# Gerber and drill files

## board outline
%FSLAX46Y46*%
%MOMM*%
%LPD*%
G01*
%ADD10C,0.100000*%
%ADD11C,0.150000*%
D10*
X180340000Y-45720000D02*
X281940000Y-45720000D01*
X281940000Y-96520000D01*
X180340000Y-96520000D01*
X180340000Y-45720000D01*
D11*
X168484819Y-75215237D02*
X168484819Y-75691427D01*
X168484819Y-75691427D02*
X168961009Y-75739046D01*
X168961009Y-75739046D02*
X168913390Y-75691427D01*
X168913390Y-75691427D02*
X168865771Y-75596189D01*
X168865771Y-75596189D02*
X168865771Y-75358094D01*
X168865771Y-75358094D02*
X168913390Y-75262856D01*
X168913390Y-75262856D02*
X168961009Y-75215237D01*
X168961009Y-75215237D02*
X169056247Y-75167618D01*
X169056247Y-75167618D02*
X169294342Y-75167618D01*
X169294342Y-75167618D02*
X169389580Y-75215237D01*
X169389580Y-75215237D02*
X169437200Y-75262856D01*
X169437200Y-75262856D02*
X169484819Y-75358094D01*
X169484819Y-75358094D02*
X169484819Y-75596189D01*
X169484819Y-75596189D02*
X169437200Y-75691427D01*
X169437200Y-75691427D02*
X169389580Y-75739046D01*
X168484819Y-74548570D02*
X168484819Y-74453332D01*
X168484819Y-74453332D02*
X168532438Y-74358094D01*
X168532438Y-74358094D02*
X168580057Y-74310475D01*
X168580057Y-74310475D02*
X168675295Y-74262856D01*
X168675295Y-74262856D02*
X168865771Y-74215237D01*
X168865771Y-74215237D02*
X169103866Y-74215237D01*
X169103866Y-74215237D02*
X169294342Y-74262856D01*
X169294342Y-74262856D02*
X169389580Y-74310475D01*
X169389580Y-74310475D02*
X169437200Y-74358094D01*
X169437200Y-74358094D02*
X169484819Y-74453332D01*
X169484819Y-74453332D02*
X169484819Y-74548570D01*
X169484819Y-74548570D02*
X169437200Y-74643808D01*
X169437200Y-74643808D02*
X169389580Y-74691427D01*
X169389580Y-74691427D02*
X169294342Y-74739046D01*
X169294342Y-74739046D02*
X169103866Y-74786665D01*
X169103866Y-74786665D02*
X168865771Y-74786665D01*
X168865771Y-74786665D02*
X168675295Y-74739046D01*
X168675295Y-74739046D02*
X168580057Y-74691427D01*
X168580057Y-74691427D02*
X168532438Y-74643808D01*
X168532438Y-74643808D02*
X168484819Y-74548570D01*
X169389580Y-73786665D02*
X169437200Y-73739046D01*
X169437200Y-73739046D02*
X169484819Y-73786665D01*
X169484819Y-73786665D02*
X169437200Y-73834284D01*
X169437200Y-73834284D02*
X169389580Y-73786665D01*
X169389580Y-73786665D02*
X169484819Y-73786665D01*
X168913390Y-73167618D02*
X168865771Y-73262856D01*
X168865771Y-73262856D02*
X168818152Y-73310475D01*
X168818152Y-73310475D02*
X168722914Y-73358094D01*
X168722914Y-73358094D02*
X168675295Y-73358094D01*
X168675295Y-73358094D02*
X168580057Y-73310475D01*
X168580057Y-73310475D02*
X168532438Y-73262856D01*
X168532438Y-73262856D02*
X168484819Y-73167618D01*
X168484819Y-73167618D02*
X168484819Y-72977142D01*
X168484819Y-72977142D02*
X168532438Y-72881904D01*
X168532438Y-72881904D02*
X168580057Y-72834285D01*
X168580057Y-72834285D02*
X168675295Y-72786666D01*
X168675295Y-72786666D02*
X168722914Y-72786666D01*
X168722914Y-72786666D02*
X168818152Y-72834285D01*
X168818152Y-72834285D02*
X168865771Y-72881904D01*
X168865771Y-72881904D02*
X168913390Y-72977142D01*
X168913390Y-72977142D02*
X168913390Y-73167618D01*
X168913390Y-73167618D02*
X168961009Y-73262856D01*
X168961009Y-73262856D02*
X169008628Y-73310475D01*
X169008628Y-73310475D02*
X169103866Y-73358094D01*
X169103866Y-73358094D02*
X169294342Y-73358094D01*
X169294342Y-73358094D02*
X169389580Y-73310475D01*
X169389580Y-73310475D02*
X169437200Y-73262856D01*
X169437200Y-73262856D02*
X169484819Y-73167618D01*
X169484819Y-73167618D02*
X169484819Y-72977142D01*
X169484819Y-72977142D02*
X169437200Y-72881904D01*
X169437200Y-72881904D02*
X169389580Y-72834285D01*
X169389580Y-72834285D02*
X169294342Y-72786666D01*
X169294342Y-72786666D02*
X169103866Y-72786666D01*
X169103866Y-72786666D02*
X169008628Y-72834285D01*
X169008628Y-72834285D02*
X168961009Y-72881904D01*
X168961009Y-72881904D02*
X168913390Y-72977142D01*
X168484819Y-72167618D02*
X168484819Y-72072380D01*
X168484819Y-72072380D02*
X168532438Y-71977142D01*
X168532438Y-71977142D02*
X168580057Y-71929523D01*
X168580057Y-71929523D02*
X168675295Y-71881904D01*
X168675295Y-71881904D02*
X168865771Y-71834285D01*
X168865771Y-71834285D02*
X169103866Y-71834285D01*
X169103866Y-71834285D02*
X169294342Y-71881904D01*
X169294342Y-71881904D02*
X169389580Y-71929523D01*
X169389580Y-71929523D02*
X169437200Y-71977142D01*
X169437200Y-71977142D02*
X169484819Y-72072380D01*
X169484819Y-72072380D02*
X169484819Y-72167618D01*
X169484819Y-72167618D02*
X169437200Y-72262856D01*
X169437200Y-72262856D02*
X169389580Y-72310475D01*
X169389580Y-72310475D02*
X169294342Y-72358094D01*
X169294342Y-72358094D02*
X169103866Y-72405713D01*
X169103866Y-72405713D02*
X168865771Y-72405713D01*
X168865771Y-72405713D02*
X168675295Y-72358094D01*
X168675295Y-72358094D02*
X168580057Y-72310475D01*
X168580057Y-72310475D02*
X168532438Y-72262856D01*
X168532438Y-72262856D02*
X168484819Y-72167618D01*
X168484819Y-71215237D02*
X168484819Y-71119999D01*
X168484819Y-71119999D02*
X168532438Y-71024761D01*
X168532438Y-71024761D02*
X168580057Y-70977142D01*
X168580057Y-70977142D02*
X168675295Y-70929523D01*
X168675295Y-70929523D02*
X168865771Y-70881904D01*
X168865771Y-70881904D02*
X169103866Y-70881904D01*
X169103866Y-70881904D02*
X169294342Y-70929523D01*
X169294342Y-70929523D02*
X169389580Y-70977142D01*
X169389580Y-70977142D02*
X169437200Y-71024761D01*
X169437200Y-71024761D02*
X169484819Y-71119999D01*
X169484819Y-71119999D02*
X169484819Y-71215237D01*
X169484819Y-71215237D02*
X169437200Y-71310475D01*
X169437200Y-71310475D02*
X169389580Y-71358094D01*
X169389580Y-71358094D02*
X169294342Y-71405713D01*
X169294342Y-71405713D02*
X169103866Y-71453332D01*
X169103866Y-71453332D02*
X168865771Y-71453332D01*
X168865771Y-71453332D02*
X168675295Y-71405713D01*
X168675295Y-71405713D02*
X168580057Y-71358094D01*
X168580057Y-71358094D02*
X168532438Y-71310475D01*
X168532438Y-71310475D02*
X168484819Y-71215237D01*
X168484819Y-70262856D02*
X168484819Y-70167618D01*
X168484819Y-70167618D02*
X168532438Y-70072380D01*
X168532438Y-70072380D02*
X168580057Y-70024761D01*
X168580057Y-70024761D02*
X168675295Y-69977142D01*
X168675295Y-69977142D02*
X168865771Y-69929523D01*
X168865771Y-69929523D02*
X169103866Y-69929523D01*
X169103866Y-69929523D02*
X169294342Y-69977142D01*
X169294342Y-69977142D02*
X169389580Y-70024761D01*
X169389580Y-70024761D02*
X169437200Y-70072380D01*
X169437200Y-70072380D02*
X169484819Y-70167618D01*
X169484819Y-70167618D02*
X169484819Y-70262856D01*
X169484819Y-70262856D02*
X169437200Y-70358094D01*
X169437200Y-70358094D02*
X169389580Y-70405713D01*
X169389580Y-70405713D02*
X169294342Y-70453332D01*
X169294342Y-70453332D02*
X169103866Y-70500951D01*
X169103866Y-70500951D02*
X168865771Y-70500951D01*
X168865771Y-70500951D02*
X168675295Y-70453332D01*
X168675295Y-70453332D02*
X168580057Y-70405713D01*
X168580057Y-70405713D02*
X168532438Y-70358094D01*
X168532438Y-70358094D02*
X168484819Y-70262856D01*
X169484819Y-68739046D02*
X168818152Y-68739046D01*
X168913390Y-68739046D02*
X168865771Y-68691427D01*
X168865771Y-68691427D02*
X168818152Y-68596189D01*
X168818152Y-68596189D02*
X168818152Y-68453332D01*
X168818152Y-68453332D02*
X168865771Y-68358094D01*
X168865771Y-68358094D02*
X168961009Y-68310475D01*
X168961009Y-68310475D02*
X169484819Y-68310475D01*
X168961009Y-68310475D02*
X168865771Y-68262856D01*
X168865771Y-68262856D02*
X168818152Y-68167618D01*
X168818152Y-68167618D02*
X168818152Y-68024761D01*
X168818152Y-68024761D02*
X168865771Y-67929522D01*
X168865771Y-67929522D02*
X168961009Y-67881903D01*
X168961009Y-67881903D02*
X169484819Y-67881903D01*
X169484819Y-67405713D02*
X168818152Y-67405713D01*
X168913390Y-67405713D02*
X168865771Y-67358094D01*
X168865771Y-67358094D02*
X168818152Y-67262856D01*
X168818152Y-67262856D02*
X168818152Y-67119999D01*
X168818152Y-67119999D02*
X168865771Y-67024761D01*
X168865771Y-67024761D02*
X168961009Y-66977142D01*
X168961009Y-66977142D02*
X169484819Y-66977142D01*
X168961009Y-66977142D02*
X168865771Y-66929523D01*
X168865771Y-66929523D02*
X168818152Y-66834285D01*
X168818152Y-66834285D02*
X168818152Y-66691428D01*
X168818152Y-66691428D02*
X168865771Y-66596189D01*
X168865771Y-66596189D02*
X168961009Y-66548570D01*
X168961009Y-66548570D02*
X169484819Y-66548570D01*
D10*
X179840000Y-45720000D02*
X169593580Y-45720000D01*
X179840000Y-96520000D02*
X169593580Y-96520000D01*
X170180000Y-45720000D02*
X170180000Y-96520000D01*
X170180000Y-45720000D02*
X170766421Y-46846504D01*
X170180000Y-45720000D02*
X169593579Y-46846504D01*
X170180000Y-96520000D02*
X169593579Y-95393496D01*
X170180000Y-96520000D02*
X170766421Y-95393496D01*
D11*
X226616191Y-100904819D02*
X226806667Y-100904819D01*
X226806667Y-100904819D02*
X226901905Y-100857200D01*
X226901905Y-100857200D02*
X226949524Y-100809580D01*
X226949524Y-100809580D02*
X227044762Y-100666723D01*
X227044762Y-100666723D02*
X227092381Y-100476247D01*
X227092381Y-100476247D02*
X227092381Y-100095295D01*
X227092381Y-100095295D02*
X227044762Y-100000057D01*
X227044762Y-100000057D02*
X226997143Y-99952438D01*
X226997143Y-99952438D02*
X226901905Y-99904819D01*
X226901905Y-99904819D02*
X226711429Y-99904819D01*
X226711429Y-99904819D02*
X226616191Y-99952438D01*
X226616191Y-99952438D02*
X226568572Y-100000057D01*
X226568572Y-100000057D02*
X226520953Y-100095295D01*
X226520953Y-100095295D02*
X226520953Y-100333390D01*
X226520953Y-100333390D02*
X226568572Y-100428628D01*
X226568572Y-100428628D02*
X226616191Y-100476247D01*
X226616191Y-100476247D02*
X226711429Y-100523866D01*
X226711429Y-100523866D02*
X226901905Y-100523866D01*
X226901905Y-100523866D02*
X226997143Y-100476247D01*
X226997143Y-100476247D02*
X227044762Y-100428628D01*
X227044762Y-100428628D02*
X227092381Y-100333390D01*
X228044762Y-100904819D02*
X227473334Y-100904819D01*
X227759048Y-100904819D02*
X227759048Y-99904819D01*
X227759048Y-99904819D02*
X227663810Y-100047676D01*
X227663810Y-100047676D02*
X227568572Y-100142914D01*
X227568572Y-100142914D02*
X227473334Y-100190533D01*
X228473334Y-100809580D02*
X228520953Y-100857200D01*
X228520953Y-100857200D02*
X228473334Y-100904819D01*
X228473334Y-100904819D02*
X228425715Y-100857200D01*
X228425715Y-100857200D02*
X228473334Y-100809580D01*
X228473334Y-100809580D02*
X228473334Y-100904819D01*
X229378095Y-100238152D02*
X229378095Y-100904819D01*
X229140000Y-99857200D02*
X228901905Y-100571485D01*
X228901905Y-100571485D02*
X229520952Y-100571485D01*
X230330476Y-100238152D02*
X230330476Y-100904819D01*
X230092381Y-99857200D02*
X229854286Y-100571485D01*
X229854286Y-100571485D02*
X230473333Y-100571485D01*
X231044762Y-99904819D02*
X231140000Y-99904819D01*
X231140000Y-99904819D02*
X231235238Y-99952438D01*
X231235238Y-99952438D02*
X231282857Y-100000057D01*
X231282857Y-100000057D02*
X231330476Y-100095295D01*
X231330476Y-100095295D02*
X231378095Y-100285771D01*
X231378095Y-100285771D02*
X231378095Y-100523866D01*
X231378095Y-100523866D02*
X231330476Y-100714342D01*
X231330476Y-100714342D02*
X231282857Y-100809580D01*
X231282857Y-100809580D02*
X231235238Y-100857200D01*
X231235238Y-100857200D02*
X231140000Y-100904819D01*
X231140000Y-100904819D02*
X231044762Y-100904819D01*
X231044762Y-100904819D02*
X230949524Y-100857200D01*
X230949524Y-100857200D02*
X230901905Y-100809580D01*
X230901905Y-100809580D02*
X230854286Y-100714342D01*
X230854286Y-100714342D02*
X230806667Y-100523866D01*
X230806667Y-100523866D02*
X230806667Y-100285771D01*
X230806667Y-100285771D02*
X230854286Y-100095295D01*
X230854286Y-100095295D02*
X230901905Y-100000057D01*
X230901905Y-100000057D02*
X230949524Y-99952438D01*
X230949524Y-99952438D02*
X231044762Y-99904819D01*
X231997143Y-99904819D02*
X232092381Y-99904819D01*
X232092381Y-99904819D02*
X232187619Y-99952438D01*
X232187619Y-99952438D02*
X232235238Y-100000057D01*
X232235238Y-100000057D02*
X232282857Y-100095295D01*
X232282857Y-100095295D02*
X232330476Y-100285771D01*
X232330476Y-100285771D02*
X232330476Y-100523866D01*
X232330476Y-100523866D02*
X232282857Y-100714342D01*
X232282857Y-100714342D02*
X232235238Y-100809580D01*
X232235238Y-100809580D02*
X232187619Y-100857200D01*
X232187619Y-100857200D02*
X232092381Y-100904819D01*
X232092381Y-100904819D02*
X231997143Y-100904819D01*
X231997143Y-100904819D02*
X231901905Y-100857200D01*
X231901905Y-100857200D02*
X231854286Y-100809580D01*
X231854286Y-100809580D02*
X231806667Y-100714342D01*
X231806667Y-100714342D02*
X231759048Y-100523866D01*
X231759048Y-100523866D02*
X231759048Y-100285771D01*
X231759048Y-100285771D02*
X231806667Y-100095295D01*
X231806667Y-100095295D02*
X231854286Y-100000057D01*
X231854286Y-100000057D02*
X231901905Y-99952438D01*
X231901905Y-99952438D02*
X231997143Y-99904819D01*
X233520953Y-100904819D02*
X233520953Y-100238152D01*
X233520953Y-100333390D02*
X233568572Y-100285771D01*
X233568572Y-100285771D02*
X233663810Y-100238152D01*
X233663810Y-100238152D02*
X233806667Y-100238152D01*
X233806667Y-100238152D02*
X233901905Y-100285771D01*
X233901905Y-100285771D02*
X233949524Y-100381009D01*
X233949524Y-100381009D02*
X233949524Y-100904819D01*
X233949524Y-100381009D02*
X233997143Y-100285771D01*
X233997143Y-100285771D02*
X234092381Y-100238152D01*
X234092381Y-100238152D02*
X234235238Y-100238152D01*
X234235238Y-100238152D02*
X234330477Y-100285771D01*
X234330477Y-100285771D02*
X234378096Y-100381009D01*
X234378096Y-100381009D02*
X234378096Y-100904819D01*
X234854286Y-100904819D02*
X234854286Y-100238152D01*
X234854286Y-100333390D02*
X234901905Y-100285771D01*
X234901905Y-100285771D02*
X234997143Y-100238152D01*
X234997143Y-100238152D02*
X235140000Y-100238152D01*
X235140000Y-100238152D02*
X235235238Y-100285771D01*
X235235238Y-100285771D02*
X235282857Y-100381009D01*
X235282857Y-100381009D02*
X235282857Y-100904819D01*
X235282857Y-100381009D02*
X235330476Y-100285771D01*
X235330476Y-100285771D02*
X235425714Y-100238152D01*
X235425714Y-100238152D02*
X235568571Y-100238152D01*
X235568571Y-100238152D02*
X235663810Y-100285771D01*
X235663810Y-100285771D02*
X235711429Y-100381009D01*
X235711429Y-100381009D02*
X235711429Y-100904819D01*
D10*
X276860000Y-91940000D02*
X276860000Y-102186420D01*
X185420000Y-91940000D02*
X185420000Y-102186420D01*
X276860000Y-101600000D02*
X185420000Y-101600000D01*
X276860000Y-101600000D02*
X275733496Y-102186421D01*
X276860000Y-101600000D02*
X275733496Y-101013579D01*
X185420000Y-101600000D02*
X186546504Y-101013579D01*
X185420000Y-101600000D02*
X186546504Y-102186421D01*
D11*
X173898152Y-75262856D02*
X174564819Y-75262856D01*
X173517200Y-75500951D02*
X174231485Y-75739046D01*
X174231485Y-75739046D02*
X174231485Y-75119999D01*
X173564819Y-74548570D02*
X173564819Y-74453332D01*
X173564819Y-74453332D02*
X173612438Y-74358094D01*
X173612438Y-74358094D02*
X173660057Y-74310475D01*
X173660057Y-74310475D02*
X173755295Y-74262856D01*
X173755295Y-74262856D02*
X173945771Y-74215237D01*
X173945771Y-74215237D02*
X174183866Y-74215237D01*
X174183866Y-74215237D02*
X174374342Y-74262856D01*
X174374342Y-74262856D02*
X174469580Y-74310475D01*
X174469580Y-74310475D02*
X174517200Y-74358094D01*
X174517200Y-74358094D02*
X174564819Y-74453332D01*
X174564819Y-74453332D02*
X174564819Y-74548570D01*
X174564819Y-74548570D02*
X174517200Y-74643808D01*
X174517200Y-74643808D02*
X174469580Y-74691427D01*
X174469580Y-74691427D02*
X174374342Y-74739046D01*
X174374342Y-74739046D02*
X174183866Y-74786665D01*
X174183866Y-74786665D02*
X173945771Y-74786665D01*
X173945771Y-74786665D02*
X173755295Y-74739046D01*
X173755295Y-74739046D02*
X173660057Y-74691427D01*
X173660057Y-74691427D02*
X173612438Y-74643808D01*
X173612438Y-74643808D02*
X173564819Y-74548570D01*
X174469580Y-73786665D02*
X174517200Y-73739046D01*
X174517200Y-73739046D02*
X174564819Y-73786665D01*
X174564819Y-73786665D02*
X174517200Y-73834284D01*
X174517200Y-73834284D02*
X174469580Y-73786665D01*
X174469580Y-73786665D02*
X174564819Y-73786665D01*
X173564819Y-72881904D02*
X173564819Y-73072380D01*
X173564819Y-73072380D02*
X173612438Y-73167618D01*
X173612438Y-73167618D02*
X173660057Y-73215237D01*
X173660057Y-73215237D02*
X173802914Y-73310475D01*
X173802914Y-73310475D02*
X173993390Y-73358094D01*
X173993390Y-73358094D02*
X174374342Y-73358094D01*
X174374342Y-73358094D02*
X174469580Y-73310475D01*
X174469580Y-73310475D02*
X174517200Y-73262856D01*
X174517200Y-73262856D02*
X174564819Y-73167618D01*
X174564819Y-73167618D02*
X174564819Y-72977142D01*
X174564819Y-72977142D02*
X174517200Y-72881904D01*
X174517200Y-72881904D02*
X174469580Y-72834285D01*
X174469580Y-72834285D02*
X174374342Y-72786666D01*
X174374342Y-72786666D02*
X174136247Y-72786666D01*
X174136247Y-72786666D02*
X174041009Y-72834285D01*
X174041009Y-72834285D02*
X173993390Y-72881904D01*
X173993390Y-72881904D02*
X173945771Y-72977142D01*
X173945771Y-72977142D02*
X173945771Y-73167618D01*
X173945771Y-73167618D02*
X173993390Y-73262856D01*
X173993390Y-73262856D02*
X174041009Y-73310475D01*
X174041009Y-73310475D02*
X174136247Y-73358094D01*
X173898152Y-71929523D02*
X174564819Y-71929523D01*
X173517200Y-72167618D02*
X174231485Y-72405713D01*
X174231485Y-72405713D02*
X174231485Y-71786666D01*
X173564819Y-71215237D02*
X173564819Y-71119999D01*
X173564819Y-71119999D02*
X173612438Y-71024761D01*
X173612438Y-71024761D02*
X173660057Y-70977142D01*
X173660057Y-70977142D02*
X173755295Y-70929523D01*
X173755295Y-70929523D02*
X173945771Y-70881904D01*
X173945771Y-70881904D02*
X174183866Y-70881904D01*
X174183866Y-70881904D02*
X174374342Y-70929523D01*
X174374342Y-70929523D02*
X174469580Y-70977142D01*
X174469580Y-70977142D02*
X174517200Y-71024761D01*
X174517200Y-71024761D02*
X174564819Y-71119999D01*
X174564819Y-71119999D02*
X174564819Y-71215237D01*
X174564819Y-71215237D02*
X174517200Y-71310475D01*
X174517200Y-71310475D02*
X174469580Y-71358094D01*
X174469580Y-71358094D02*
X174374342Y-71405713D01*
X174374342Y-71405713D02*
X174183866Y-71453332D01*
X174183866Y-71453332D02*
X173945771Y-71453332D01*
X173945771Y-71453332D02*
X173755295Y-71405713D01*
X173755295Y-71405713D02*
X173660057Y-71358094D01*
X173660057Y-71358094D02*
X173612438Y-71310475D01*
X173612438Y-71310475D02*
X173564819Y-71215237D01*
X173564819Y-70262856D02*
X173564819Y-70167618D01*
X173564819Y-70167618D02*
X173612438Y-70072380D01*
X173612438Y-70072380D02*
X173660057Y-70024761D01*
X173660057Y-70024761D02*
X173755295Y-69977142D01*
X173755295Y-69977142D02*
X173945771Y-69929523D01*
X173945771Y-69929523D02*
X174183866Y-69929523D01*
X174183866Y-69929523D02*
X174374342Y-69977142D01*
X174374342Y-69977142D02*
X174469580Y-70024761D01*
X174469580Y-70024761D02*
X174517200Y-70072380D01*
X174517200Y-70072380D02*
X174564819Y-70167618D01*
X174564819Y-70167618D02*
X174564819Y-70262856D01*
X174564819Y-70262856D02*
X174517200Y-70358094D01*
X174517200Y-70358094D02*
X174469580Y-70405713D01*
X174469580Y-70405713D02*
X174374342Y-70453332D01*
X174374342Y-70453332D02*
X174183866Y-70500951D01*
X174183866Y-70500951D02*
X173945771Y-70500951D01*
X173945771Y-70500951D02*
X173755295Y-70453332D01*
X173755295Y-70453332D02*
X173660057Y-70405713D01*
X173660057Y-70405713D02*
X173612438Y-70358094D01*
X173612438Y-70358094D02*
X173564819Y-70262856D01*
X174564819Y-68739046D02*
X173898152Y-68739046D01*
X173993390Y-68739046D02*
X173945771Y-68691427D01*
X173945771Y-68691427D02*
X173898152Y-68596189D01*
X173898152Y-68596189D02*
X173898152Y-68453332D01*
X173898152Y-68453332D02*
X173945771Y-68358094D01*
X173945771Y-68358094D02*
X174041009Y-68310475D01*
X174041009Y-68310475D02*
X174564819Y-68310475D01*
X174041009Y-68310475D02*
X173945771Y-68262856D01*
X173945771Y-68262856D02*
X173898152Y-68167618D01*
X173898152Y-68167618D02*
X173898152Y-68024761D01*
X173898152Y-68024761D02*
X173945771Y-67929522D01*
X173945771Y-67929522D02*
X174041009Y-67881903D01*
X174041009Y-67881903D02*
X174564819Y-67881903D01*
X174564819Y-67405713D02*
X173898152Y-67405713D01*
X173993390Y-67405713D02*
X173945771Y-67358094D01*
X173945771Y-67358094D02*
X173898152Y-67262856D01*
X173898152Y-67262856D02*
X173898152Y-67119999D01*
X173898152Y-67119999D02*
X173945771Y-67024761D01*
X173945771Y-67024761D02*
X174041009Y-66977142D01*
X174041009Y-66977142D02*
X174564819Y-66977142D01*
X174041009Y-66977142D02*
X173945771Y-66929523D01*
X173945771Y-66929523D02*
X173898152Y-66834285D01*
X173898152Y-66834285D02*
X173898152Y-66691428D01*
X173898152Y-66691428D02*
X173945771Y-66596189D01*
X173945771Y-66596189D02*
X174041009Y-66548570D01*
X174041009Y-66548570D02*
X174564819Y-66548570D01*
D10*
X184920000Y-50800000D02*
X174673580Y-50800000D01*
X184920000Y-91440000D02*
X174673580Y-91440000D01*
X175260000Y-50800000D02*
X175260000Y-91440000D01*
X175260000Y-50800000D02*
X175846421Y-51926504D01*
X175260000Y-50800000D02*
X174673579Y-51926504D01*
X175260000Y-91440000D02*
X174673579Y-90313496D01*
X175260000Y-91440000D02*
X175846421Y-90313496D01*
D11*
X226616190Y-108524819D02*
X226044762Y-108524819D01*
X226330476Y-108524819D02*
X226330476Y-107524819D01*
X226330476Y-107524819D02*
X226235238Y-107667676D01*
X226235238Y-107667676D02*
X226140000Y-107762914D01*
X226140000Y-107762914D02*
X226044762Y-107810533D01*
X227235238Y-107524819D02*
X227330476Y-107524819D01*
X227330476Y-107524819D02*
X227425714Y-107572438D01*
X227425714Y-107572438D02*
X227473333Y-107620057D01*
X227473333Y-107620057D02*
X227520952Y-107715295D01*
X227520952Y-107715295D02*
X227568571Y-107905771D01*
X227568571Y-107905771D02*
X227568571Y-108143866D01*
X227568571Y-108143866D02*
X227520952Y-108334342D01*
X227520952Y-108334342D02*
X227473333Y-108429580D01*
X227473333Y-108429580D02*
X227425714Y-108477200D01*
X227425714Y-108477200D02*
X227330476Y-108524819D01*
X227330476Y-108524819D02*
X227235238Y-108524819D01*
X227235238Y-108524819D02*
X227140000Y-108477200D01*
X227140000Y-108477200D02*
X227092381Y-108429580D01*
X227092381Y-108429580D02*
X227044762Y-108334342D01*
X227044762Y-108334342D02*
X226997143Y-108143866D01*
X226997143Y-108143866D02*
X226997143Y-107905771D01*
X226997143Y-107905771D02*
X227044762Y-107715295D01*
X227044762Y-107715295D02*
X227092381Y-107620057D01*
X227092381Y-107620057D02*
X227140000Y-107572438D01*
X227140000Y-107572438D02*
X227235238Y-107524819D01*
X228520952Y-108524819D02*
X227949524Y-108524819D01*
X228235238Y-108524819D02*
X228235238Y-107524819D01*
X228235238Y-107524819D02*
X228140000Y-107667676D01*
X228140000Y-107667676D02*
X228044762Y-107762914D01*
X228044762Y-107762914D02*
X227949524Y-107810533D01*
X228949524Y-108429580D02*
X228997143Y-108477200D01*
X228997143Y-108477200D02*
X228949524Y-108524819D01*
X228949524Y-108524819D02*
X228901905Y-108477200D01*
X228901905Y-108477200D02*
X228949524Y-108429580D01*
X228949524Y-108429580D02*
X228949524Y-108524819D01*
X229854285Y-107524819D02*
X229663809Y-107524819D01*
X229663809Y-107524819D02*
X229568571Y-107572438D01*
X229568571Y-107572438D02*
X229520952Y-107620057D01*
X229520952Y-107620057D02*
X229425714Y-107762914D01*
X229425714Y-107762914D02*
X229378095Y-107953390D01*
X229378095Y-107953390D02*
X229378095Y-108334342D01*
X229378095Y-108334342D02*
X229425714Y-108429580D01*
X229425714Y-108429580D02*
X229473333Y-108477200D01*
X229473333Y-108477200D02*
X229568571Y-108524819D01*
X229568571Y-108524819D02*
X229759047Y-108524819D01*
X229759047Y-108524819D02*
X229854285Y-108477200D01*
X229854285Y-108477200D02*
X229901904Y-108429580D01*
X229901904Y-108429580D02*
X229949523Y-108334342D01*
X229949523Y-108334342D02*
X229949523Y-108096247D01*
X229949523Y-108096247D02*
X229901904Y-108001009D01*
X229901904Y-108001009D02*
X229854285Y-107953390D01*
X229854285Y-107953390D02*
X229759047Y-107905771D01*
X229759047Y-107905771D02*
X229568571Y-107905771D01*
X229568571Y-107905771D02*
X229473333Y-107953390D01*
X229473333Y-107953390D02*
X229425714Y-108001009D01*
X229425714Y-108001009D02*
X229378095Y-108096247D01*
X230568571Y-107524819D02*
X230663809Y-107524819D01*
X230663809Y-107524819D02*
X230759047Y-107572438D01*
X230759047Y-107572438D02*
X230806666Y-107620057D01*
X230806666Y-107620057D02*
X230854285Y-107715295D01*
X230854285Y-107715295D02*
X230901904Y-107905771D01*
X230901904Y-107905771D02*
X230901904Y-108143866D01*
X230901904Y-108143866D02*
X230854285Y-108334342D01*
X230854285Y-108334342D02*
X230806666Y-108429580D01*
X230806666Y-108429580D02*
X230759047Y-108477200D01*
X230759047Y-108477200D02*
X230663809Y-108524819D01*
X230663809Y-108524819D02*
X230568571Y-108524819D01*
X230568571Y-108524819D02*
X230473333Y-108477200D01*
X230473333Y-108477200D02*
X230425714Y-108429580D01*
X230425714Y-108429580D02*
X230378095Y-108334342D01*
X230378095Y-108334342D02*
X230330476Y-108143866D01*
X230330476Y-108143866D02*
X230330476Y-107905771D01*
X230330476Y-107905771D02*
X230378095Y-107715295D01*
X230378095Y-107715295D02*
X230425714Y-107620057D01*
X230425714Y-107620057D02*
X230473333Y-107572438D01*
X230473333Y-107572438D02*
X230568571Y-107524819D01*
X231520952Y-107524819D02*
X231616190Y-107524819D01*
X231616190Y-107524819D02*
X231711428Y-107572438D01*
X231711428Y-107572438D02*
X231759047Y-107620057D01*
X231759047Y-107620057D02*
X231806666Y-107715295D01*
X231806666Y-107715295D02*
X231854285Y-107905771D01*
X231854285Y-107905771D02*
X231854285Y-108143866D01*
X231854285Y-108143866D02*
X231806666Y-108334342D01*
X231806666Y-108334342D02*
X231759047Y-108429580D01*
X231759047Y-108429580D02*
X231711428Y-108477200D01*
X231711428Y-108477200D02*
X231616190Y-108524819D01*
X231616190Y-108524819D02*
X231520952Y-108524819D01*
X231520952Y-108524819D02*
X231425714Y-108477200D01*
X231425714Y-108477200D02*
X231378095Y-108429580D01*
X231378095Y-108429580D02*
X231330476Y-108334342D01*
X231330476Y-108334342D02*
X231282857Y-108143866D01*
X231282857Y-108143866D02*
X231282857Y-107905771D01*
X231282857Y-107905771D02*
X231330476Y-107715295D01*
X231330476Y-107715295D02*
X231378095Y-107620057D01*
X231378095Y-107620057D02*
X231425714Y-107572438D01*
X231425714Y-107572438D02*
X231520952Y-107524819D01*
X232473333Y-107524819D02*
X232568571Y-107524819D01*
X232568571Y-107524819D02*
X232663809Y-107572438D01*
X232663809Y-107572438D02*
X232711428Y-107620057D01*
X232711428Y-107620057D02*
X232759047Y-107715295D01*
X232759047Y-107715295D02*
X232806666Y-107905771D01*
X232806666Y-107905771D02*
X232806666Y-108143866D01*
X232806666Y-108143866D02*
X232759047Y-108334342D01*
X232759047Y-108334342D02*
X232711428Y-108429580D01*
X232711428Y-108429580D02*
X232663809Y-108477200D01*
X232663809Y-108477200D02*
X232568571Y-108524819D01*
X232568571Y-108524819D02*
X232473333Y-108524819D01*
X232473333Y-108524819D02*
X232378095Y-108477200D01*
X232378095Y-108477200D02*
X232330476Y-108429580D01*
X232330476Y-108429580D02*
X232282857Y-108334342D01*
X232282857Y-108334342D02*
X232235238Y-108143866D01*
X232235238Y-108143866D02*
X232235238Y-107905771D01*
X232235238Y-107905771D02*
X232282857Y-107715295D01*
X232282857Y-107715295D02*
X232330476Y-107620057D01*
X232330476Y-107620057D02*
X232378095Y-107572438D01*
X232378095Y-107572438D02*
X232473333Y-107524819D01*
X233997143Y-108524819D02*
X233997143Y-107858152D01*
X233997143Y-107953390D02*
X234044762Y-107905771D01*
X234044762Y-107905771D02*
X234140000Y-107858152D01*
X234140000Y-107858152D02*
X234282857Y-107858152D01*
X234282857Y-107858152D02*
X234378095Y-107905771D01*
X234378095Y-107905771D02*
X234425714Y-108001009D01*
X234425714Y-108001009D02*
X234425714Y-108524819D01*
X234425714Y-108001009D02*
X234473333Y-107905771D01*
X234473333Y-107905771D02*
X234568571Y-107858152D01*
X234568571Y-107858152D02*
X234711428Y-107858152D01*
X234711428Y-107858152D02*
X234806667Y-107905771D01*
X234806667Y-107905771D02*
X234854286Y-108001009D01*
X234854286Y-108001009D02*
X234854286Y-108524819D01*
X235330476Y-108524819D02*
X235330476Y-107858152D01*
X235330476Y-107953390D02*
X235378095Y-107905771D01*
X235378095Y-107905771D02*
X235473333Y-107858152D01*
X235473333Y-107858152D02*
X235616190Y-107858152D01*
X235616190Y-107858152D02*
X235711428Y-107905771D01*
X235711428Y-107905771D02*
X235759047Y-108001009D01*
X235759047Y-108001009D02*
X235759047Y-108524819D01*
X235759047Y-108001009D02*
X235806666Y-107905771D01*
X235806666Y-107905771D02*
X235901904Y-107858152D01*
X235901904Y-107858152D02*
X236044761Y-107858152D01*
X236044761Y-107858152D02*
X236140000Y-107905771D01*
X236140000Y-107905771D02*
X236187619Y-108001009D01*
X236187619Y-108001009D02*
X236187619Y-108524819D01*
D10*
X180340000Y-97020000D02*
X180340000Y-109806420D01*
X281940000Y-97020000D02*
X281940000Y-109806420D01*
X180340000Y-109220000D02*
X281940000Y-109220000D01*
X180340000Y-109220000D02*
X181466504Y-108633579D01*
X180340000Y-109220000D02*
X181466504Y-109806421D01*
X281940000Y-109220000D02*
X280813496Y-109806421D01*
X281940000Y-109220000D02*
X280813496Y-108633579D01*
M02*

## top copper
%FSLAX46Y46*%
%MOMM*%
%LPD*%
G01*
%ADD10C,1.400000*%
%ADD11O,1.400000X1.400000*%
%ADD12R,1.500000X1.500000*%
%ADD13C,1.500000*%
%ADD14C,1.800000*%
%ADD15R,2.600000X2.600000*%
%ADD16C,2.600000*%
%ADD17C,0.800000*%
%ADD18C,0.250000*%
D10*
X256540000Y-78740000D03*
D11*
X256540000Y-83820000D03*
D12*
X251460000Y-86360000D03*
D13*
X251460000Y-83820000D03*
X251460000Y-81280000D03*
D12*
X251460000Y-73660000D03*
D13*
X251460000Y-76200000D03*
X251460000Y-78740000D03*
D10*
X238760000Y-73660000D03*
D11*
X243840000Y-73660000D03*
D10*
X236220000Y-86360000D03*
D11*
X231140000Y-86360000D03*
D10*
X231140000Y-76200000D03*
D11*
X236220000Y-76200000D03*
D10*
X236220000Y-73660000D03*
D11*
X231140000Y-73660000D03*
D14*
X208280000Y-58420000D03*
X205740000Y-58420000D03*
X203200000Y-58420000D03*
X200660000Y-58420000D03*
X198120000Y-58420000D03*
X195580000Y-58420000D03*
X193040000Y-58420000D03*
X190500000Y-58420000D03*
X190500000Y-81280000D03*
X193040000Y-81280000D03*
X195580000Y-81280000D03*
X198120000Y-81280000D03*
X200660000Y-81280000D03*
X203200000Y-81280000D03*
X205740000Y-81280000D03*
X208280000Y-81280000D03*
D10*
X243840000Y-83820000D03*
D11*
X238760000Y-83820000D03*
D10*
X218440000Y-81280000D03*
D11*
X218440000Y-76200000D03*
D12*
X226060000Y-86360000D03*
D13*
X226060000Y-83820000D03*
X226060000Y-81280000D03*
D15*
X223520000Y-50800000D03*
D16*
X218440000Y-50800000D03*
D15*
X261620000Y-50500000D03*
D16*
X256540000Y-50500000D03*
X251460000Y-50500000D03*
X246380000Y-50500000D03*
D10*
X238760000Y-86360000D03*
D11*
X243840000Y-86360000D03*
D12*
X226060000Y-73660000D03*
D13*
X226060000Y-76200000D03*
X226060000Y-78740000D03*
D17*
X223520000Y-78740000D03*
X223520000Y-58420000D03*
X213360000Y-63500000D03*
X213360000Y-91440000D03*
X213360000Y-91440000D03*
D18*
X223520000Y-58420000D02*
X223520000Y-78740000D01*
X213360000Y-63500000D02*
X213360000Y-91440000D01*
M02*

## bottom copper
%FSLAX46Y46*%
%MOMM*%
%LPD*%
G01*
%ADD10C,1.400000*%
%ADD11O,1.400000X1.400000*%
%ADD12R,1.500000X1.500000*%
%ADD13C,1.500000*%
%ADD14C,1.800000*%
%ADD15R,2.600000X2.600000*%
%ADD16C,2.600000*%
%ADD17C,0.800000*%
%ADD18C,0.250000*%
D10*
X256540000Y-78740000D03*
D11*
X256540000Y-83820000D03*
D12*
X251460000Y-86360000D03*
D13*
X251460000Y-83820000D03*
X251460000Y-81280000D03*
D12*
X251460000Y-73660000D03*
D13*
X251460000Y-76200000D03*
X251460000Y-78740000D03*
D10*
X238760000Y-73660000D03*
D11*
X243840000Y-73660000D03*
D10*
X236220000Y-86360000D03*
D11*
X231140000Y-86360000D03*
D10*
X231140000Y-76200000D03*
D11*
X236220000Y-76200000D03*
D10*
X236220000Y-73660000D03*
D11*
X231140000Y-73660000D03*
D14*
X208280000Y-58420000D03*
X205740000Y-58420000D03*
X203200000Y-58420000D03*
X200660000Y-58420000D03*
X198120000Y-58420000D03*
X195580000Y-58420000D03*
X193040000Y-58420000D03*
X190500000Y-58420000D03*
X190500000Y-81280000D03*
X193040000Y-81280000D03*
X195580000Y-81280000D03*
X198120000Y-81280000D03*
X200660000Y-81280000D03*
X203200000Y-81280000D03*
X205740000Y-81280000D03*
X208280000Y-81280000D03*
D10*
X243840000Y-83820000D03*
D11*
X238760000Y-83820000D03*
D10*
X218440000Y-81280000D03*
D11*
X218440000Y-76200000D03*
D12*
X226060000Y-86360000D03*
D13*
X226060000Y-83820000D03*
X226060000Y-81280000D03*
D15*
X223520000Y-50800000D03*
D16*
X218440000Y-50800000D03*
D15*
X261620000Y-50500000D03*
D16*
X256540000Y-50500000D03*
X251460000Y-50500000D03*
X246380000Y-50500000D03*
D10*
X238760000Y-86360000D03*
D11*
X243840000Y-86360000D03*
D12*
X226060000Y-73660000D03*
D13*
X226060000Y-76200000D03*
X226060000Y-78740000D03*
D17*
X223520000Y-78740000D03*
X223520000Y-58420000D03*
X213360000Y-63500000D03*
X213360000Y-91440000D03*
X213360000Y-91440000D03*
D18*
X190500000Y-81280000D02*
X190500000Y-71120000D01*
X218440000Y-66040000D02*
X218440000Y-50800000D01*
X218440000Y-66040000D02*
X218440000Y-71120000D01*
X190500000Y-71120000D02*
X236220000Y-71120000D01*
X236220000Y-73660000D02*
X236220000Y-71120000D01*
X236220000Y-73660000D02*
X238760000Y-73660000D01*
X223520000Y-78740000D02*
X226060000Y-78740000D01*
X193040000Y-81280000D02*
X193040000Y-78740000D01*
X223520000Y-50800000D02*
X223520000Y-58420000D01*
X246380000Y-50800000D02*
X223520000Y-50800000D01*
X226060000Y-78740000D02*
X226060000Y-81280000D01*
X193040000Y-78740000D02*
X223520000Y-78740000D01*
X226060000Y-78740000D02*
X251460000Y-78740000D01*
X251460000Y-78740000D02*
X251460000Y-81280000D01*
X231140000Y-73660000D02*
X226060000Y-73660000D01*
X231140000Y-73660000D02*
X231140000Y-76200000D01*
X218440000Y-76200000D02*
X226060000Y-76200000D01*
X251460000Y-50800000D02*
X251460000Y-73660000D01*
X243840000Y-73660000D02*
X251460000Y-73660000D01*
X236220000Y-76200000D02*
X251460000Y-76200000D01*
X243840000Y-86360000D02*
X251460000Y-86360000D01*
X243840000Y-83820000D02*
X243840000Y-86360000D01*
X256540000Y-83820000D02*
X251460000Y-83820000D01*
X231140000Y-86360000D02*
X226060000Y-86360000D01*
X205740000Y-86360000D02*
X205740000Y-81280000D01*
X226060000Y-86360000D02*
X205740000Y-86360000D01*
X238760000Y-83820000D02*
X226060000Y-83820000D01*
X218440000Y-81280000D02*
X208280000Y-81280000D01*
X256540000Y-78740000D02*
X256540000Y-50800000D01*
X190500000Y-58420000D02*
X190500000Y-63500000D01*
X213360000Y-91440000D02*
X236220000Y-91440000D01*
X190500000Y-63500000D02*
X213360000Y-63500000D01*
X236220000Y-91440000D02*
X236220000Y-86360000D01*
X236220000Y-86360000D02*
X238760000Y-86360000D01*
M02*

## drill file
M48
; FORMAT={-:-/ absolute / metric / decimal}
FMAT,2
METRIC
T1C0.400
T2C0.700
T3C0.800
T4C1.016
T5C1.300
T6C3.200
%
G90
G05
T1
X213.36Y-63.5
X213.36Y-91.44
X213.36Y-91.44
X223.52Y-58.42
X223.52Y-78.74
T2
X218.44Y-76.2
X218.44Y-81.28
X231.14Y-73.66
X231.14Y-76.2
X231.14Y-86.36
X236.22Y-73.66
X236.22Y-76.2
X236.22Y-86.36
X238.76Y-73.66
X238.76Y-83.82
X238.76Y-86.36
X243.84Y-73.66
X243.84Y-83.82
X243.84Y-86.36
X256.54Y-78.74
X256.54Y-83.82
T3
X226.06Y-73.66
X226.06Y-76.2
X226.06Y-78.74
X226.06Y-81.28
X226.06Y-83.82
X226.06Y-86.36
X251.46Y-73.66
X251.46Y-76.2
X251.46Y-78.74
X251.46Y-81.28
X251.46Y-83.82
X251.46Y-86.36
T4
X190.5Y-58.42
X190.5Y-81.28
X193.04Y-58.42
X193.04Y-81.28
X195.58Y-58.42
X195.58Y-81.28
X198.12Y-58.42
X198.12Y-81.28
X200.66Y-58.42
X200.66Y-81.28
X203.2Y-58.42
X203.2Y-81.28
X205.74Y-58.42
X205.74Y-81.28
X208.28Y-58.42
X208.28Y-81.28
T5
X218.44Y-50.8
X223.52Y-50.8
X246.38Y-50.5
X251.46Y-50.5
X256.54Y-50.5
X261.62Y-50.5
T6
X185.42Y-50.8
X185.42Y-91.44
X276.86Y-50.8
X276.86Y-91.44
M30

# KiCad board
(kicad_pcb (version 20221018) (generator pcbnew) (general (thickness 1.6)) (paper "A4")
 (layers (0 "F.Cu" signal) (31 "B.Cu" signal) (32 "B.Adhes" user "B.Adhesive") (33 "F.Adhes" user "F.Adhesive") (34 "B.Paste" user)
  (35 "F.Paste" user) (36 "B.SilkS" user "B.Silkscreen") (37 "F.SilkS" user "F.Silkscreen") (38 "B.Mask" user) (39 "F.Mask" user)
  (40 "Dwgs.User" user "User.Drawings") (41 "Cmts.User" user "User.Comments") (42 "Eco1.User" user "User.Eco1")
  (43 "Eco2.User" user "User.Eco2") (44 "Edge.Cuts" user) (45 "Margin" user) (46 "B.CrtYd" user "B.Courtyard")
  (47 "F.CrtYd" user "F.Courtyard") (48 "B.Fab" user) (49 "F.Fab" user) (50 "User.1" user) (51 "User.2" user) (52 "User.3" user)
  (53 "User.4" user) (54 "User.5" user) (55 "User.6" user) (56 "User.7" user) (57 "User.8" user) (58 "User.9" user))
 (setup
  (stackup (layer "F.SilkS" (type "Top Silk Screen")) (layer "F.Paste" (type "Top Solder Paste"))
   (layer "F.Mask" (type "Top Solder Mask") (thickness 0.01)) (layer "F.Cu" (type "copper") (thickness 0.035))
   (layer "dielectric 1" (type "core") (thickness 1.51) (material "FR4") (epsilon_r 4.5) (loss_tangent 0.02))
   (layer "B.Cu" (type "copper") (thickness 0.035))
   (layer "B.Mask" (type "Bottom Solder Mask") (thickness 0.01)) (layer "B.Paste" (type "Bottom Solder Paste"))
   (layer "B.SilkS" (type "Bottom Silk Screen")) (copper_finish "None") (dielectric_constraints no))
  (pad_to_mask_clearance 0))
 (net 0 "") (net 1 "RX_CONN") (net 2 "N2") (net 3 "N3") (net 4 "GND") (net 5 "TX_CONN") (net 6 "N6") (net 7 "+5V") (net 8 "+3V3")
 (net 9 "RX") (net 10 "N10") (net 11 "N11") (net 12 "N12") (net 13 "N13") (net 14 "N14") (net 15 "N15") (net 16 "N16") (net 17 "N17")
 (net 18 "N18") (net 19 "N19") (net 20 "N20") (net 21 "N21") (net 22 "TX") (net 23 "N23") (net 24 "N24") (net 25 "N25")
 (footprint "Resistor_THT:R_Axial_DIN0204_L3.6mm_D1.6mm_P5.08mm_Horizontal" (layer "F.Cu") (at 256.54 78.74 -90)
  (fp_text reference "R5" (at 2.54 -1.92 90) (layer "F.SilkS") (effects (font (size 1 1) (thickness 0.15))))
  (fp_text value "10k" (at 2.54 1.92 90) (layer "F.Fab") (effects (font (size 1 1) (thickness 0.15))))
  (pad "1" thru_hole circle (at 0 0 270) (size 1.4 1.4) (drill 0.7) (layers "*.Cu" "*.Mask") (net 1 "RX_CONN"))
  (pad "2" thru_hole oval (at 5.08 0 270) (size 1.4 1.4) (drill 0.7) (layers "*.Cu" "*.Mask") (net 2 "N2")))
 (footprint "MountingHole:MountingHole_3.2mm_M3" (layer "F.Cu") (at 185.42 91.44)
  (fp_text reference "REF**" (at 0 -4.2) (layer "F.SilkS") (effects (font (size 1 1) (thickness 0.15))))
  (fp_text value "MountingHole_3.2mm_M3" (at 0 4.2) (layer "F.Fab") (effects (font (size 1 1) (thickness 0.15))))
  (pad "" np_thru_hole circle (at 0 0) (size 3.2 3.2) (drill 3.2) (layers "*.Cu" "*.Mask")))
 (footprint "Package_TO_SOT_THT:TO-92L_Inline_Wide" (layer "F.Cu") (at 251.46 86.36 90)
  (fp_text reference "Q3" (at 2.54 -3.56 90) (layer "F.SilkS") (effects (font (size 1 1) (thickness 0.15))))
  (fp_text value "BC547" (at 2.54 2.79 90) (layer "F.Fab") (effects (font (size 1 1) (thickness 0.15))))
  (pad "1" thru_hole rect (at 0 0 90) (size 1.5 1.5) (drill 0.8) (layers "*.Cu" "*.Mask") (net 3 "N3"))
  (pad "2" thru_hole circle (at 2.54 0 90) (size 1.5 1.5) (drill 0.8) (layers "*.Cu" "*.Mask") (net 2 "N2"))
  (pad "3" thru_hole circle (at 5.08 0 90) (size 1.5 1.5) (drill 0.8) (layers "*.Cu" "*.Mask") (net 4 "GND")))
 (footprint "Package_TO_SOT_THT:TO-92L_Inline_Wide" (layer "F.Cu") (at 251.46 73.66 -90)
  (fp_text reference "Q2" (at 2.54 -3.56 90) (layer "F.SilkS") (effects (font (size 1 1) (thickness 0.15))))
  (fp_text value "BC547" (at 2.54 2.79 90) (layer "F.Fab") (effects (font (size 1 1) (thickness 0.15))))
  (pad "1" thru_hole rect (at 0 0 270) (size 1.5 1.5) (drill 0.8) (layers "*.Cu" "*.Mask") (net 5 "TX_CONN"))
  (pad "2" thru_hole circle (at 2.54 0 270) (size 1.5 1.5) (drill 0.8) (layers "*.Cu" "*.Mask") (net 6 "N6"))
  (pad "3" thru_hole circle (at 5.08 0 270) (size 1.5 1.5) (drill 0.8) (layers "*.Cu" "*.Mask") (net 4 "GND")))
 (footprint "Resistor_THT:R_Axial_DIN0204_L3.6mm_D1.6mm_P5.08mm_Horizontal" (layer "F.Cu") (at 238.76 73.66)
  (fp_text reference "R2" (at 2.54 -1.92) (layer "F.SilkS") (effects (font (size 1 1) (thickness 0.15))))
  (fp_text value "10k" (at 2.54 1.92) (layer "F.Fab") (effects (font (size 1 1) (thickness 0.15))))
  (pad "1" thru_hole circle (at 0 0) (size 1.4 1.4) (drill 0.7) (layers "*.Cu" "*.Mask") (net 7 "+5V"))
  (pad "2" thru_hole oval (at 5.08 0) (size 1.4 1.4) (drill 0.7) (layers "*.Cu" "*.Mask") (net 5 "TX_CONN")))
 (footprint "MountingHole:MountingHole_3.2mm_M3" (layer "F.Cu") (at 276.86 91.44)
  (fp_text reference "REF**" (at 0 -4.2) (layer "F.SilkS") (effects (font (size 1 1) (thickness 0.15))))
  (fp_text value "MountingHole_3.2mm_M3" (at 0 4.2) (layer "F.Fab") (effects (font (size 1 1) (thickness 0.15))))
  (pad "" np_thru_hole circle (at 0 0) (size 3.2 3.2) (drill 3.2) (layers "F&B.Cu" "*.Mask")))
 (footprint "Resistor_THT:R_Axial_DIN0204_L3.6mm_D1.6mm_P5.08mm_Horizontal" (layer "F.Cu") (at 236.22 86.36 180)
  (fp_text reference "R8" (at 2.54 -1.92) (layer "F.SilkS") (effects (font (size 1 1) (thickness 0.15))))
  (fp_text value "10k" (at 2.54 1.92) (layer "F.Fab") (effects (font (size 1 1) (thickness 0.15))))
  (pad "1" thru_hole circle (at 0 0 180) (size 1.4 1.4) (drill 0.7) (layers "*.Cu" "*.Mask") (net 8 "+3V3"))
  (pad "2" thru_hole oval (at 5.08 0 180) (size 1.4 1.4) (drill 0.7) (layers "*.Cu" "*.Mask") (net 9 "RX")))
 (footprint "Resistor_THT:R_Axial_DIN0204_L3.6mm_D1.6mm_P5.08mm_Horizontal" (layer "F.Cu") (at 231.14 76.2)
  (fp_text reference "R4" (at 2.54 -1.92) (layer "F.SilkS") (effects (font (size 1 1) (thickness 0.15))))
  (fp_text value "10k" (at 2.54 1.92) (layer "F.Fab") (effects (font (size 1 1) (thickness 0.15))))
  (pad "1" thru_hole circle (at 0 0) (size 1.4 1.4) (drill 0.7) (layers "*.Cu" "*.Mask") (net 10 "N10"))
  (pad "2" thru_hole oval (at 5.08 0) (size 1.4 1.4) (drill 0.7) (layers "*.Cu" "*.Mask") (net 6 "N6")))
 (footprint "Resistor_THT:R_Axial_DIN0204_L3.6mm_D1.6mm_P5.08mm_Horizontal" (layer "F.Cu") (at 236.22 73.66 180)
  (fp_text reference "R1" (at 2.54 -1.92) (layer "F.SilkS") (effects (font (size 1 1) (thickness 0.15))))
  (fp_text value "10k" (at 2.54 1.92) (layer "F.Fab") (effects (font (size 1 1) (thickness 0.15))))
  (pad "1" thru_hole circle (at 0 0 180) (size 1.4 1.4) (drill 0.7) (layers "*.Cu" "*.Mask") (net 7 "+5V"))
  (pad "2" thru_hole oval (at 5.08 0 180) (size 1.4 1.4) (drill 0.7) (layers "*.Cu" "*.Mask") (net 10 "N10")))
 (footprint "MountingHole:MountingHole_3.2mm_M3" (layer "F.Cu") (at 185.42 50.8)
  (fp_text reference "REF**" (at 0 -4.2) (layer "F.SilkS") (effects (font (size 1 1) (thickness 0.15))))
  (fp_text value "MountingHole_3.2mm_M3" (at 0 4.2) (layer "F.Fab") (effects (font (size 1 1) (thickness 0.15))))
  (pad "" np_thru_hole circle (at 0 0) (size 3.2 3.2) (drill 3.2) (layers "F&B.Cu" "*.Mask")))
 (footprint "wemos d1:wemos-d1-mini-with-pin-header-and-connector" (layer "F.Cu") (at 199.39 69.85)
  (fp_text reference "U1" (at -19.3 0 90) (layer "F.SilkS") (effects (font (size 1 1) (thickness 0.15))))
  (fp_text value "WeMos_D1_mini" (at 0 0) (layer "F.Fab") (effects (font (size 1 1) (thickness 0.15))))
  (pad "1" thru_hole circle (at 8.89 -11.43) (size 1.8 1.8) (drill 1.016) (layers "*.Cu" "*.Mask") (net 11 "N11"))
  (pad "2" thru_hole circle (at 6.35 -11.43) (size 1.8 1.8) (drill 1.016) (layers "*.Cu" "*.Mask") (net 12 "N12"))
  (pad "3" thru_hole circle (at 3.81 -11.43) (size 1.8 1.8) (drill 1.016) (layers "*.Cu" "*.Mask") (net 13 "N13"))
  (pad "4" thru_hole circle (at 1.27 -11.43) (size 1.8 1.8) (drill 1.016) (layers "*.Cu" "*.Mask") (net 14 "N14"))
  (pad "5" thru_hole circle (at -1.27 -11.43) (size 1.8 1.8) (drill 1.016) (layers "*.Cu" "*.Mask") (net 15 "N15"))
  (pad "6" thru_hole circle (at -3.81 -11.43 90) (size 1.8 1.8) (drill 1.016) (layers "*.Cu" "*.Mask") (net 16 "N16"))
  (pad "7" thru_hole circle (at -6.35 -11.43) (size 1.8 1.8) (drill 1.016) (layers "*.Cu" "*.Mask") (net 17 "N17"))
  (pad "8" thru_hole circle (at -8.89 -11.43) (size 1.8 1.8) (drill 1.016) (layers "*.Cu" "*.Mask") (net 8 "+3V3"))
  (pad "9" thru_hole circle (at -8.89 11.43) (size 1.8 1.8) (drill 1.016) (layers "*.Cu" "*.Mask") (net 7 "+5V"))
  (pad "10" thru_hole circle (at -6.35 11.43) (size 1.8 1.8) (drill 1.016) (layers "*.Cu" "*.Mask") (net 4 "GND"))
  (pad "11" thru_hole circle (at -3.81 11.43) (size 1.8 1.8) (drill 1.016) (layers "*.Cu" "*.Mask") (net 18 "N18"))
  (pad "12" thru_hole circle (at -1.27 11.43) (size 1.8 1.8) (drill 1.016) (layers "*.Cu" "*.Mask") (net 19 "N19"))
  (pad "13" thru_hole circle (at 1.27 11.43) (size 1.8 1.8) (drill 1.016) (layers "*.Cu" "*.Mask") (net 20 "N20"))
  (pad "14" thru_hole circle (at 3.81 11.43) (size 1.8 1.8) (drill 1.016) (layers "*.Cu" "*.Mask") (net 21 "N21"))
  (pad "15" thru_hole circle (at 6.35 11.43) (size 1.8 1.8) (drill 1.016) (layers "*.Cu" "*.Mask") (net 9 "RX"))
  (pad "16" thru_hole circle (at 8.89 11.43) (size 1.8 1.8) (drill 1.016) (layers "*.Cu" "*.Mask") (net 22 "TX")))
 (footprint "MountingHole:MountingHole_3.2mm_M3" (layer "F.Cu") (at 276.86 50.8)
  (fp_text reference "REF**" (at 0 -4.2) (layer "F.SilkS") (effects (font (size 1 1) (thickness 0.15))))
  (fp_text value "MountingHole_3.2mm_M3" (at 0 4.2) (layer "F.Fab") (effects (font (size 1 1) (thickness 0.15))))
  (pad "" np_thru_hole circle (at 0 0) (size 3.2 3.2) (drill 3.2) (layers "F&B.Cu" "*.Mask")))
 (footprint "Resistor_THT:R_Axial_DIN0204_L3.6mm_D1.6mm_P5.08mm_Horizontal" (layer "F.Cu") (at 243.84 83.82 180)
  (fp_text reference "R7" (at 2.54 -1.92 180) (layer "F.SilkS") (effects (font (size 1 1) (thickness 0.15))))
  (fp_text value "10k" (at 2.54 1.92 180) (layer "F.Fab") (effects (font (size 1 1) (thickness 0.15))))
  (pad "1" thru_hole circle (at 0 0 180) (size 1.4 1.4) (drill 0.7) (layers "*.Cu" "*.Mask") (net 3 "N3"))
  (pad "2" thru_hole oval (at 5.08 0 180) (size 1.4 1.4) (drill 0.7) (layers "*.Cu" "*.Mask") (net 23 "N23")))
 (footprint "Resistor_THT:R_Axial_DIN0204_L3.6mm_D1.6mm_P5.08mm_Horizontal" (layer "F.Cu") (at 218.44 81.28 90)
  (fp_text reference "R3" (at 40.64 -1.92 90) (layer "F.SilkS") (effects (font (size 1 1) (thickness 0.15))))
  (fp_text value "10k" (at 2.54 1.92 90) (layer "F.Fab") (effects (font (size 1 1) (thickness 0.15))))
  (pad "1" thru_hole circle (at 0 0 90) (size 1.4 1.4) (drill 0.7) (layers "*.Cu" "*.Mask") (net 22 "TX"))
  (pad "2" thru_hole oval (at 5.08 0 90) (size 1.4 1.4) (drill 0.7) (layers "*.Cu" "*.Mask") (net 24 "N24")))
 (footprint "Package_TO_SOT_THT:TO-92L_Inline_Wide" (layer "F.Cu") (at 226.06 86.36 90)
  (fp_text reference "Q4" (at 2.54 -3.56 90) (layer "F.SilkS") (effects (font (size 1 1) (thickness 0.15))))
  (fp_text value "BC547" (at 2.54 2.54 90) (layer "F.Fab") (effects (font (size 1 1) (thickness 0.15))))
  (pad "1" thru_hole rect (at 0 0 90) (size 1.5 1.5) (drill 0.8) (layers "*.Cu" "*.Mask") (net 9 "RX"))
  (pad "2" thru_hole circle (at 2.54 0 90) (size 1.5 1.5) (drill 0.8) (layers "*.Cu" "*.Mask") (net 23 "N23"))
  (pad "3" thru_hole circle (at 5.08 0 90) (size 1.5 1.5) (drill 0.8) (layers "*.Cu" "*.Mask") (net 4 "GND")))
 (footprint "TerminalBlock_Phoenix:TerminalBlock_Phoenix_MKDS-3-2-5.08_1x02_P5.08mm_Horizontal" (layer "F.Cu") (at 223.52 50.8 180)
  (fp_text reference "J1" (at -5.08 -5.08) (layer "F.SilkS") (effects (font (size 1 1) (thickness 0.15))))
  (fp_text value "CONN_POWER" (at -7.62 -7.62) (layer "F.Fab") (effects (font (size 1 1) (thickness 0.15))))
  (pad "1" thru_hole rect (at 0 0 180) (size 2.6 2.6) (drill 1.3) (layers "*.Cu" "*.Mask") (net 4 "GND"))
  (pad "2" thru_hole circle (at 5.08 0 180) (size 2.6 2.6) (drill 1.3) (layers "*.Cu" "*.Mask") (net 7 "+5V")))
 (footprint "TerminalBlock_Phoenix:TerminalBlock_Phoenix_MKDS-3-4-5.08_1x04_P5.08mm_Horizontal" (layer "F.Cu") (at 261.62 50.5 180)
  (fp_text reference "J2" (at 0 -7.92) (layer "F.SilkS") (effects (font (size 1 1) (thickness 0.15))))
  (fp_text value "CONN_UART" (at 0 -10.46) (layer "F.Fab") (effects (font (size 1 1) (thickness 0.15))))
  (pad "1" thru_hole rect (at 0 0 180) (size 2.6 2.6) (drill 1.3) (layers "*.Cu" "*.Mask") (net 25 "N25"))
  (pad "2" thru_hole circle (at 5.08 0 180) (size 2.6 2.6) (drill 1.3) (layers "*.Cu" "*.Mask") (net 1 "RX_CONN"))
  (pad "3" thru_hole circle (at 10.16 0 180) (size 2.6 2.6) (drill 1.3) (layers "*.Cu" "*.Mask") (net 5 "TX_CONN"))
  (pad "4" thru_hole circle (at 15.24 0 180) (size 2.6 2.6) (drill 1.3) (layers "*.Cu" "*.Mask") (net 4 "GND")))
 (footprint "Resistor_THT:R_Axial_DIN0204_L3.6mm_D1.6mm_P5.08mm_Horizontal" (layer "F.Cu") (at 238.76 86.36)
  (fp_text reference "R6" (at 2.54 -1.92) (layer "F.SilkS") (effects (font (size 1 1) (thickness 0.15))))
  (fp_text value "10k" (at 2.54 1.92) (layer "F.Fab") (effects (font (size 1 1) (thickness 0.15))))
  (pad "1" thru_hole circle (at 0 0) (size 1.4 1.4) (drill 0.7) (layers "*.Cu" "*.Mask") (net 8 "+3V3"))
  (pad "2" thru_hole oval (at 5.08 0) (size 1.4 1.4) (drill 0.7) (layers "*.Cu" "*.Mask") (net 3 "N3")))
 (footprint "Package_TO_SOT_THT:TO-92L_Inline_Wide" (layer "F.Cu") (at 226.06 73.66 -90)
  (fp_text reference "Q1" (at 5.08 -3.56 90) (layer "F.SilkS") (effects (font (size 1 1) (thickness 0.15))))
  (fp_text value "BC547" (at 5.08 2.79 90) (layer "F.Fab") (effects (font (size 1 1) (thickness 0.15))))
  (pad "1" thru_hole rect (at 0 0 270) (size 1.5 1.5) (drill 0.8) (layers "*.Cu" "*.Mask") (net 10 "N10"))
  (pad "2" thru_hole circle (at 2.54 0 270) (size 1.5 1.5) (drill 0.8) (layers "*.Cu" "*.Mask") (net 24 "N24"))
  (pad "3" thru_hole circle (at 5.08 0 270) (size 1.5 1.5) (drill 0.8) (layers "*.Cu" "*.Mask") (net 4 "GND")))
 (gr_rect (start 180.34 45.72) (end 281.94 96.52) (stroke (width 0.1) (type default)) (fill none) (layer "Edge.Cuts"))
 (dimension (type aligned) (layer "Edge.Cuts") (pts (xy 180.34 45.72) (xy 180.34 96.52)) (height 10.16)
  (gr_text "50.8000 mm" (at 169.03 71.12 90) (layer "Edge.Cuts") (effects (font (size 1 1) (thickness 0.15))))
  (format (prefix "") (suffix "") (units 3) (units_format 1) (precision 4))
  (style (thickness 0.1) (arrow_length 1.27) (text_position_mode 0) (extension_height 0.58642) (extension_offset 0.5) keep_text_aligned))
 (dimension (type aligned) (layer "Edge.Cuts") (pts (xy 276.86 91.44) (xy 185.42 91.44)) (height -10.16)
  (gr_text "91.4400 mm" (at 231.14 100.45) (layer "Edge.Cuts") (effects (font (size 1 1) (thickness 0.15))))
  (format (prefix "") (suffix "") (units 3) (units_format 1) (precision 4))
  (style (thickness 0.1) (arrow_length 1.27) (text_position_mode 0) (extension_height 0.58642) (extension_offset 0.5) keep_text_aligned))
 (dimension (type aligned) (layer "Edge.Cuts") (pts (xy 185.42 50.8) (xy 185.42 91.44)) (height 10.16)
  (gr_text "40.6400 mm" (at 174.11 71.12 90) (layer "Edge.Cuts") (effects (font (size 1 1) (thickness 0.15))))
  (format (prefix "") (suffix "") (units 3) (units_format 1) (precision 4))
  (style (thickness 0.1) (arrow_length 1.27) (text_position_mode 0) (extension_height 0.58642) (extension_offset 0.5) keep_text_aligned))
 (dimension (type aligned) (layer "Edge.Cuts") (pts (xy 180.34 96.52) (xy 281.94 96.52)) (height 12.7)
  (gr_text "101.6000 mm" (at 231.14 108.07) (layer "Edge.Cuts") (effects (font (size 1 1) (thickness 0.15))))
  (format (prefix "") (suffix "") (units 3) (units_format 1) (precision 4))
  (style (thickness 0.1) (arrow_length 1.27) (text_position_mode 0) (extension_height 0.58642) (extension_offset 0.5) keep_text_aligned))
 (segment (start 190.5 81.28) (end 190.5 71.12) (width 0.25) (layer "B.Cu") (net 7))
 (segment (start 218.44 66.04) (end 218.44 50.8) (width 0.25) (layer "B.Cu") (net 7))
 (segment (start 218.44 66.04) (end 218.44 71.12) (width 0.25) (layer "B.Cu") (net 7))
 (segment (start 190.5 71.12) (end 236.22 71.12) (width 0.25) (layer "B.Cu") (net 7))
 (segment (start 236.22 73.66) (end 236.22 71.12) (width 0.25) (layer "B.Cu") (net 7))
 (segment (start 236.22 73.66) (end 238.76 73.66) (width 0.25) (layer "B.Cu") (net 7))
 (segment (start 223.52 58.42) (end 223.52 78.74) (width 0.25) (layer "F.Cu") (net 4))
 (via (at 223.52 78.74) (size 0.8) (drill 0.4) (layers "F.Cu" "B.Cu") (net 4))
 (via (at 223.52 58.42) (size 0.8) (drill 0.4) (layers "F.Cu" "B.Cu") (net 4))
 (segment (start 223.52 78.74) (end 226.06 78.74) (width 0.25) (layer "B.Cu") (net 4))
 (segment (start 193.04 81.28) (end 193.04 78.74) (width 0.25) (layer "B.Cu") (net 4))
 (segment (start 223.52 50.8) (end 223.52 58.42) (width 0.25) (layer "B.Cu") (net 4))
 (segment (start 246.38 50.8) (end 223.52 50.8) (width 0.25) (layer "B.Cu") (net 4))
 (segment (start 226.06 78.74) (end 226.06 81.28) (width 0.25) (layer "B.Cu") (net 4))
 (segment (start 193.04 78.74) (end 223.52 78.74) (width 0.25) (layer "B.Cu") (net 4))
 (segment (start 226.06 78.74) (end 251.46 78.74) (width 0.25) (layer "B.Cu") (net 4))
 (segment (start 251.46 78.74) (end 251.46 81.28) (width 0.25) (layer "B.Cu") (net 4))
 (segment (start 231.14 73.66) (end 226.06 73.66) (width 0.25) (layer "B.Cu") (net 10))
 (segment (start 231.14 73.66) (end 231.14 76.2) (width 0.25) (layer "B.Cu") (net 10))
 (segment (start 218.44 76.2) (end 226.06 76.2) (width 0.25) (layer "B.Cu") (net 24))
 (segment (start 251.46 50.8) (end 251.46 73.66) (width 0.25) (layer "B.Cu") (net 5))
 (segment (start 243.84 73.66) (end 251.46 73.66) (width 0.25) (layer "B.Cu") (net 5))
 (segment (start 236.22 76.2) (end 251.46 76.2) (width 0.25) (layer "B.Cu") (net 6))
 (segment (start 243.84 86.36) (end 251.46 86.36) (width 0.25) (layer "B.Cu") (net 3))
 (segment (start 243.84 83.82) (end 243.84 86.36) (width 0.25) (layer "B.Cu") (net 3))
 (segment (start 256.54 83.82) (end 251.46 83.82) (width 0.25) (layer "B.Cu") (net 2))
 (segment (start 231.14 86.36) (end 226.06 86.36) (width 0.25) (layer "B.Cu") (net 9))
 (segment (start 205.74 86.36) (end 205.74 81.28) (width 0.25) (layer "B.Cu") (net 9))
 (segment (start 226.06 86.36) (end 205.74 86.36) (width 0.25) (layer "B.Cu") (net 9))
 (segment (start 238.76 83.82) (end 226.06 83.82) (width 0.25) (layer "B.Cu") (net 23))
 (segment (start 218.44 81.28) (end 208.28 81.28) (width 0.25) (layer "B.Cu") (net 22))
 (segment (start 256.54 78.74) (end 256.54 50.8) (width 0.25) (layer "B.Cu") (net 1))
 (segment (start 213.36 63.5) (end 213.36 91.44) (width 0.25) (layer "F.Cu") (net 8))
 (via (at 213.36 63.5) (size 0.8) (drill 0.4) (layers "F.Cu" "B.Cu") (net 8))
 (via (at 213.36 91.44) (size 0.8) (drill 0.4) (layers "F.Cu" "B.Cu") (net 8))
 (via (at 213.36 91.44) (size 0.8) (drill 0.4) (layers "F.Cu" "B.Cu") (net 8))
 (segment (start 190.5 58.42) (end 190.5 63.5) (width 0.25) (layer "B.Cu") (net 8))
 (segment (start 213.36 91.44) (end 236.22 91.44) (width 0.25) (layer "B.Cu") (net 8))
 (segment (start 190.5 63.5) (end 213.36 63.5) (width 0.25) (layer "B.Cu") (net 8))
 (segment (start 236.22 91.44) (end 236.22 86.36) (width 0.25) (layer "B.Cu") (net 8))
 (segment (start 236.22 86.36) (end 238.76 86.36) (width 0.25) (layer "B.Cu") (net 8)))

